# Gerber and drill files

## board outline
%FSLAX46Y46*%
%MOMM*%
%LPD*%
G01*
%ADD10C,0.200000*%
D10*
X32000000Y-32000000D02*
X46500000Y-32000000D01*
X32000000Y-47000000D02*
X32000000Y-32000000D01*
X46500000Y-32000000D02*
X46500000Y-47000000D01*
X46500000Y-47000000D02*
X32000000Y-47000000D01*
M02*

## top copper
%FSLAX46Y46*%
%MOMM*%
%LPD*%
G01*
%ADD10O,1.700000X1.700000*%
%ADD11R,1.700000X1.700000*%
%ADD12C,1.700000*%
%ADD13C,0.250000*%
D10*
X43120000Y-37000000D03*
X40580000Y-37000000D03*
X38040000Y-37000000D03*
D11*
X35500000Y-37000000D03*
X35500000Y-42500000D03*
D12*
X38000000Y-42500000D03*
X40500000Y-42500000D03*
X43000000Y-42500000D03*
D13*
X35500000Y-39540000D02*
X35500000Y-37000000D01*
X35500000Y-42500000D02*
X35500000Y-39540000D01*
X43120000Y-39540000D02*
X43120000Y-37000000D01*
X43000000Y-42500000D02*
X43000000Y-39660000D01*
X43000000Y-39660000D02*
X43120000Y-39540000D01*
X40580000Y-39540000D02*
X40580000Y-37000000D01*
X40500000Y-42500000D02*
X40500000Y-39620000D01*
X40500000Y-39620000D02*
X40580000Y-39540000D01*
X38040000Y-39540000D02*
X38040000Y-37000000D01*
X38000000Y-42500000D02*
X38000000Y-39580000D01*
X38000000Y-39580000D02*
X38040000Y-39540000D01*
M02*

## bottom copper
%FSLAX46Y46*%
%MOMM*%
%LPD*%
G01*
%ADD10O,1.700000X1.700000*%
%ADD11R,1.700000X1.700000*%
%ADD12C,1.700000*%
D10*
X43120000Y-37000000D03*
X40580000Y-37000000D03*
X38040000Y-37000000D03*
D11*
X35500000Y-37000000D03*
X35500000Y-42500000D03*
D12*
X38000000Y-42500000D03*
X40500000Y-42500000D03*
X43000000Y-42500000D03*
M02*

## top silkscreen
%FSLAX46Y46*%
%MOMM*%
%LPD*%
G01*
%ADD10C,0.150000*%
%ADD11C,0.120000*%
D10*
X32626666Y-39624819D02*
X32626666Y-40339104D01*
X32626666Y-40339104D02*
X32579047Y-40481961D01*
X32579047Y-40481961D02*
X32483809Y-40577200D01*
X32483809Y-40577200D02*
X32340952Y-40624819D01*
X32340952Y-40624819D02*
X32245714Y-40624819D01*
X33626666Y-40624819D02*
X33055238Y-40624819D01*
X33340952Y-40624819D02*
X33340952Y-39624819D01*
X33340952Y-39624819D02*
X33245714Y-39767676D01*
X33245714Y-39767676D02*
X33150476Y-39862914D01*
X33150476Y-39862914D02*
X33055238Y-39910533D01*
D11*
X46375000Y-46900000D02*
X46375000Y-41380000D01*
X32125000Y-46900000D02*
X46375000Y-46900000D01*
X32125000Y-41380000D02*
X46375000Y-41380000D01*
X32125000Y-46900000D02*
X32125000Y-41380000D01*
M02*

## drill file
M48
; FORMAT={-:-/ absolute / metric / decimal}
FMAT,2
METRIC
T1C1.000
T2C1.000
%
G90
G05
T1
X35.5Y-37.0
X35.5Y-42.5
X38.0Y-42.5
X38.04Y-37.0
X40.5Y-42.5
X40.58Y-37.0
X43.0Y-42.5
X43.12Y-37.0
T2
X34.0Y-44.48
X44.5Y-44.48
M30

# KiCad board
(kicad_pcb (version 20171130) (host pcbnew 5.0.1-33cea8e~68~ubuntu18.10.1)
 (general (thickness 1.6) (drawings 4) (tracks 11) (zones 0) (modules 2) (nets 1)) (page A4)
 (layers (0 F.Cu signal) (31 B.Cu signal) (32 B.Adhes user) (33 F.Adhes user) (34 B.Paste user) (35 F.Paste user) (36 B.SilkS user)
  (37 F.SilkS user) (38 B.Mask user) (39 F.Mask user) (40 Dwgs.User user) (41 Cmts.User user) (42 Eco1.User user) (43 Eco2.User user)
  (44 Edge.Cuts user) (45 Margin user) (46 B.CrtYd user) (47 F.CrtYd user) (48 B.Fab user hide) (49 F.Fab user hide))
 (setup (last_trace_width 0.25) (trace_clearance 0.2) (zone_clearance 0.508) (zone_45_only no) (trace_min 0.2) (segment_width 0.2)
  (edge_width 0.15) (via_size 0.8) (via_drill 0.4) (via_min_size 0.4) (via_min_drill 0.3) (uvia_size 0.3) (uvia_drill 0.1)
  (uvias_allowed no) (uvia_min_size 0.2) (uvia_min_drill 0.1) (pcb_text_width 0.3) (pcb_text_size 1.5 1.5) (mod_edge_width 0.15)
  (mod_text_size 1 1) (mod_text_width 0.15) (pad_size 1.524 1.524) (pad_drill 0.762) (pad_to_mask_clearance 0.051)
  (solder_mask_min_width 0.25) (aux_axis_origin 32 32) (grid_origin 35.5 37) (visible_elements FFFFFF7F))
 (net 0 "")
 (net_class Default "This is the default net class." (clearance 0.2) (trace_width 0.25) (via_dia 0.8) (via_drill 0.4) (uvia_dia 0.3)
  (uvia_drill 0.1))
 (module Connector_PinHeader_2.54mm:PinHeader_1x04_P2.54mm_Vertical (layer B.Cu) (at 35.5 37 270)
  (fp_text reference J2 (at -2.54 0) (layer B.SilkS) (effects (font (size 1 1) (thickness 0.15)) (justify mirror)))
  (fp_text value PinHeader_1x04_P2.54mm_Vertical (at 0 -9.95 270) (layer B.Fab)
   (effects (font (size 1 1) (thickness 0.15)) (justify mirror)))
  (pad 4 thru_hole oval (at 0 -7.62 270) (size 1.7 1.7) (drill 1) (layers *.Cu *.Mask))
  (pad 3 thru_hole oval (at 0 -5.08 270) (size 1.7 1.7) (drill 1) (layers *.Cu *.Mask))
  (pad 2 thru_hole oval (at 0 -2.54 270) (size 1.7 1.7) (drill 1) (layers *.Cu *.Mask))
  (pad 1 thru_hole rect (at 0 0 270) (size 1.7 1.7) (drill 1) (layers *.Cu *.Mask)))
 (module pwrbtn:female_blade (layer F.Cu) (at 39.25 42.5)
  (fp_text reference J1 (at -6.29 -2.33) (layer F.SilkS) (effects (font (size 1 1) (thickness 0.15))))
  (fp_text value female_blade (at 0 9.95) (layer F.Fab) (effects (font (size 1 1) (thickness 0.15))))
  (fp_line (start 7.125 4.4) (end 7.125 -1.12) (layer F.SilkS) (width 0.12))
  (fp_line (start -7.125 4.4) (end 7.125 4.4) (layer F.SilkS) (width 0.12))
  (fp_line (start -7.125 -1.12) (end 7.125 -1.12) (layer F.SilkS) (width 0.12))
  (fp_line (start -7.125 4.4) (end -7.125 -1.12) (layer F.SilkS) (width 0.12))
  (pad "" np_thru_hole circle (at -5.25 1.98 90) (size 1 1) (drill 1) (layers *.Cu *.Mask))
  (pad "" np_thru_hole circle (at 5.25 1.98 90) (size 1 1) (drill 1) (layers *.Cu *.Mask))
  (pad 1 thru_hole rect (at -3.75 0 90) (size 1.7 1.7) (drill 1) (layers *.Cu *.Mask))
  (pad 2 thru_hole circle (at -1.25 0 90) (size 1.7 1.7) (drill 1) (layers *.Cu *.Mask))
  (pad 3 thru_hole circle (at 1.25 0 90) (size 1.7 1.7) (drill 1) (layers *.Cu *.Mask))
  (pad 4 thru_hole circle (at 3.75 0 90) (size 1.7 1.7) (drill 1) (layers *.Cu *.Mask)))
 (gr_line (start 32 32) (end 46.5 32) (layer Edge.Cuts) (width 0.2))
 (gr_line (start 32 47) (end 32 32) (layer Edge.Cuts) (width 0.2))
 (gr_line (start 46.5 32) (end 46.5 47) (layer Edge.Cuts) (width 0.2))
 (gr_line (start 46.5 47) (end 32 47) (layer Edge.Cuts) (width 0.2))
 (segment (start 35.5 39.54) (end 35.5 37) (width 0.25) (layer F.Cu) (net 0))
 (segment (start 35.5 42.5) (end 35.5 39.54) (width 0.25) (layer F.Cu) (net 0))
 (segment (start 43.12 39.54) (end 43.12 37) (width 0.25) (layer F.Cu) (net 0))
 (segment (start 43 42.5) (end 43 39.66) (width 0.25) (layer F.Cu) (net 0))
 (segment (start 43 39.66) (end 43.12 39.54) (width 0.25) (layer F.Cu) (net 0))
 (segment (start 40.58 39.54) (end 40.58 37) (width 0.25) (layer F.Cu) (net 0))
 (segment (start 40.5 42.5) (end 40.5 39.62) (width 0.25) (layer F.Cu) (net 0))
 (segment (start 40.5 39.62) (end 40.58 39.54) (width 0.25) (layer F.Cu) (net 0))
 (segment (start 38.04 39.54) (end 38.04 37) (width 0.25) (layer F.Cu) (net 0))
 (segment (start 38 42.5) (end 38 39.58) (width 0.25) (layer F.Cu) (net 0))
 (segment (start 38 39.58) (end 38.04 39.54) (width 0.25) (layer F.Cu) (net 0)))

